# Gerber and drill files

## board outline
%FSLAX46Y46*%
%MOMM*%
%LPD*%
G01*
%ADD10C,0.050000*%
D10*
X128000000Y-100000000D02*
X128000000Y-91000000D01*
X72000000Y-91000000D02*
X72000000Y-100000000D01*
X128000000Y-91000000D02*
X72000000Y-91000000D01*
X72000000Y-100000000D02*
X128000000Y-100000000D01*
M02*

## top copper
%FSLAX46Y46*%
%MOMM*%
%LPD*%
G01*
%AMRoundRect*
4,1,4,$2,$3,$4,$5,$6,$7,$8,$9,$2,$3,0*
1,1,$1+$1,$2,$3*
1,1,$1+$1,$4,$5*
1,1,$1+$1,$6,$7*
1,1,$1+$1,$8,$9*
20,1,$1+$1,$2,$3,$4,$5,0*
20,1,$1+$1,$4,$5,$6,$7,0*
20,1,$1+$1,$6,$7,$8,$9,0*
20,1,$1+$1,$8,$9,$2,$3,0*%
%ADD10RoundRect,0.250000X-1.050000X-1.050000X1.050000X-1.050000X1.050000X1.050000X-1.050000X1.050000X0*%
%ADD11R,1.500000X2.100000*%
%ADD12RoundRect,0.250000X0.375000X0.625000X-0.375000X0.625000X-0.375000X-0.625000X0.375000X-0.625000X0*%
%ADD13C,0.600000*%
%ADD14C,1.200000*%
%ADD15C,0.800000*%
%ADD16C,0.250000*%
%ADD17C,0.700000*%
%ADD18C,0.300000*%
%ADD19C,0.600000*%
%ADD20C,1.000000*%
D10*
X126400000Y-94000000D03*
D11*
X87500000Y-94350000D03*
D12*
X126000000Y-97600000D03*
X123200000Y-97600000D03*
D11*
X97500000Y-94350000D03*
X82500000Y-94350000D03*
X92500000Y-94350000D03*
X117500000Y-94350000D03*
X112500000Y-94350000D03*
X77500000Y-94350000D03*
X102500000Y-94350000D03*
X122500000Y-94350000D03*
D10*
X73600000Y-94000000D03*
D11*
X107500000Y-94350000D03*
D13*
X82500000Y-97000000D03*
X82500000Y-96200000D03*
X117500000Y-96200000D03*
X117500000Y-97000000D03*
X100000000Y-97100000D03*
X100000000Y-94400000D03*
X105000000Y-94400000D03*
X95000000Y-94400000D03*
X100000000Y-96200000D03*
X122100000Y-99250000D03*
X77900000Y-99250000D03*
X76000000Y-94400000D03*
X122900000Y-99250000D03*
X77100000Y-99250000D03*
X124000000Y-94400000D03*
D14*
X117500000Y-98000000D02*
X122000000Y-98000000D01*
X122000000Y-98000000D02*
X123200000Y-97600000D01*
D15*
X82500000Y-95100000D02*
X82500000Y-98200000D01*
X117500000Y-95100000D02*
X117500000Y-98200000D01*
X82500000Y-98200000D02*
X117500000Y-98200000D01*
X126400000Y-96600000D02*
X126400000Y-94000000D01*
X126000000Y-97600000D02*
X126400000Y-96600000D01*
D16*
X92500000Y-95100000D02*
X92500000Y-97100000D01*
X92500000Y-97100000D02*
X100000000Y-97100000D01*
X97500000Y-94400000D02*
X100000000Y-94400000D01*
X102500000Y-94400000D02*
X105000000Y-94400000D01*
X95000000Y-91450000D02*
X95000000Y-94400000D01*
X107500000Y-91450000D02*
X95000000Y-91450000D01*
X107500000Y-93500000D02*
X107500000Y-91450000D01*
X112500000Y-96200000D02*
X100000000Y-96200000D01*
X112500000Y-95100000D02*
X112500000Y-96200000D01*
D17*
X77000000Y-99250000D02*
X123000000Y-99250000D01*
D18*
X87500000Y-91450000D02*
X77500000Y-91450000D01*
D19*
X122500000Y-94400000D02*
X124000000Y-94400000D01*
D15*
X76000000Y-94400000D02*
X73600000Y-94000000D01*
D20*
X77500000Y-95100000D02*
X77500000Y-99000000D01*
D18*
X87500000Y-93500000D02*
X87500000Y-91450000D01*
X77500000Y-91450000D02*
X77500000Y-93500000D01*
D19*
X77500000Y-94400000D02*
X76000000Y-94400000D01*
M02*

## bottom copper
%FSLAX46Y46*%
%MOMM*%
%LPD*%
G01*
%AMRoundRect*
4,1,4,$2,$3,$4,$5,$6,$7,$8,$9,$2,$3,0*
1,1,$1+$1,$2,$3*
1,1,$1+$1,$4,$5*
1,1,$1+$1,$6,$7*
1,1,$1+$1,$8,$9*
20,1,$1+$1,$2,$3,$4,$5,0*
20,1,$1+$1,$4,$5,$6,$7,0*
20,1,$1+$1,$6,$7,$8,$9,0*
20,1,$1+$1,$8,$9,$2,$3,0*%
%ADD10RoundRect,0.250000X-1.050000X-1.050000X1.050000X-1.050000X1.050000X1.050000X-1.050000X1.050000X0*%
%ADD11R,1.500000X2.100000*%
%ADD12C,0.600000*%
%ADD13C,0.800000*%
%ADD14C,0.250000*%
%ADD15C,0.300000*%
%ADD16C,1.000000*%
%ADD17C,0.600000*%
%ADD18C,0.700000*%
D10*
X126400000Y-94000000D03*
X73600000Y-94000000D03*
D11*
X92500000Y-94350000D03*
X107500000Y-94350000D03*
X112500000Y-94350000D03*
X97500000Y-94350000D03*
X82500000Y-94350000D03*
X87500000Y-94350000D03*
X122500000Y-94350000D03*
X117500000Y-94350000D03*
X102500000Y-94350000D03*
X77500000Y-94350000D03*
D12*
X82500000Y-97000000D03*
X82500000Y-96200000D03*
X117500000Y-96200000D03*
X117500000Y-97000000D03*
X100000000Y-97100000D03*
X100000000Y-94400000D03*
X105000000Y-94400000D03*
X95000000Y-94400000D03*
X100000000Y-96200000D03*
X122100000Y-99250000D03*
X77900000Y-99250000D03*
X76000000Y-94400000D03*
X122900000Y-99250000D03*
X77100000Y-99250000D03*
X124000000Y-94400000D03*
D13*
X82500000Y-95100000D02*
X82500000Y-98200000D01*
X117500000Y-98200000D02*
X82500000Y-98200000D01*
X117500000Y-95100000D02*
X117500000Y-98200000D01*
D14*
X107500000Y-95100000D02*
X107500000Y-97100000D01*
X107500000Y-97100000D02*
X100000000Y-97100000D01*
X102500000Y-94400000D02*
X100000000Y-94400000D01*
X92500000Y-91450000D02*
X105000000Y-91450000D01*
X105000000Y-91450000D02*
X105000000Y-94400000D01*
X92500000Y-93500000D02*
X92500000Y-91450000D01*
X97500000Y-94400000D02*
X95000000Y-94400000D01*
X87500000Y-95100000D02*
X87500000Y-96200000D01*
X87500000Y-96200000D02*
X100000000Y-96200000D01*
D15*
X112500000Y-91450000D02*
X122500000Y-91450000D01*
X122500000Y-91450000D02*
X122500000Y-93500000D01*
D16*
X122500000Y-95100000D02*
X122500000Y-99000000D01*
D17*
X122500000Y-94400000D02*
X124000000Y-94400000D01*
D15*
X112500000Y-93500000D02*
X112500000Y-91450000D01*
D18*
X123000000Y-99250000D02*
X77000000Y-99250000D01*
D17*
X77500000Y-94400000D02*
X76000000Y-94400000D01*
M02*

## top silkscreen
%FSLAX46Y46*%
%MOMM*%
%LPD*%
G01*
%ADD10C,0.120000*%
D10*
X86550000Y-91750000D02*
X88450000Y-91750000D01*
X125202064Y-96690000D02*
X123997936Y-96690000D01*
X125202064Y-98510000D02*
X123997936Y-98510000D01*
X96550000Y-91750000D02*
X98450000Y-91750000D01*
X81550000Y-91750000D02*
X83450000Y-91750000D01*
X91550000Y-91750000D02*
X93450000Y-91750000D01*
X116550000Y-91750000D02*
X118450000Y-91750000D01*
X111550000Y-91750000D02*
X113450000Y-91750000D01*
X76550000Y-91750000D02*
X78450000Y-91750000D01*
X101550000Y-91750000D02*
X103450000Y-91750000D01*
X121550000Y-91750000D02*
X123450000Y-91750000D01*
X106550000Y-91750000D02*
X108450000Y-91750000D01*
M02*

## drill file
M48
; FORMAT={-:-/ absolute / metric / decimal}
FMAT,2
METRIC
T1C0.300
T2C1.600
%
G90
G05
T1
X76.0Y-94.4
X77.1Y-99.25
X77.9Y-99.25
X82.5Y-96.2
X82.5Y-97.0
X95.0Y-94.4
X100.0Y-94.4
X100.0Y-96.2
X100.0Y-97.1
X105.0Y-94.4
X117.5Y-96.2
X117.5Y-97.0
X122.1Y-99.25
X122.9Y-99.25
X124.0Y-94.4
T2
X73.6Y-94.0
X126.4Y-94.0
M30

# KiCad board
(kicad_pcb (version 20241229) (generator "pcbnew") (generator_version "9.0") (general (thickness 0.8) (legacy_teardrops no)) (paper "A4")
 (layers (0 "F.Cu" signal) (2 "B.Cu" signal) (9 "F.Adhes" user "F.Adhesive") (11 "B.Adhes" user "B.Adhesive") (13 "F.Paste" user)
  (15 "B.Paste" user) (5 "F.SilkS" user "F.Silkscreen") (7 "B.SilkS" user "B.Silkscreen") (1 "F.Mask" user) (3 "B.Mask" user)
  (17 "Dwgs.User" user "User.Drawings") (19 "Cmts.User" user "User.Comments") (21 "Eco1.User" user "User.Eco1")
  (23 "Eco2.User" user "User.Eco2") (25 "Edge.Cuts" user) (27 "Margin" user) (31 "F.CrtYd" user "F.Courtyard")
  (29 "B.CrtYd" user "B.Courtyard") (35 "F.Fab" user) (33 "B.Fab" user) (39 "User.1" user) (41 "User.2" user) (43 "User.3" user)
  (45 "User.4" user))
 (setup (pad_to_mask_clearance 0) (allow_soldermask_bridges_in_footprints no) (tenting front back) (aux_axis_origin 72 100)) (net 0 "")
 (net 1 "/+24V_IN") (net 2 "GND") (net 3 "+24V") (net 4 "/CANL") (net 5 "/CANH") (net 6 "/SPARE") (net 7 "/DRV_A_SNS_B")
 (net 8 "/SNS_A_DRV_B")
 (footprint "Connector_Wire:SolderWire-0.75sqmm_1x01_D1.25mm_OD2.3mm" (layer "F.Cu") (at 126.4 94)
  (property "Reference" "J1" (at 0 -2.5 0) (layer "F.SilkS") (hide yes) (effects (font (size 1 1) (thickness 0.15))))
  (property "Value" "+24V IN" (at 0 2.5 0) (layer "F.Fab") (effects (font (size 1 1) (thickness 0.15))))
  (pad "1" thru_hole roundrect (at 0 0) (size 2.6 2.6) (drill 1.6) (layers "*.Cu" "*.Mask") (remove_unused_layers no)
   (roundrect_rratio 0.096154) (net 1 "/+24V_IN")))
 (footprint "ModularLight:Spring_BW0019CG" (layer "F.Cu") (at 87.5 93.65)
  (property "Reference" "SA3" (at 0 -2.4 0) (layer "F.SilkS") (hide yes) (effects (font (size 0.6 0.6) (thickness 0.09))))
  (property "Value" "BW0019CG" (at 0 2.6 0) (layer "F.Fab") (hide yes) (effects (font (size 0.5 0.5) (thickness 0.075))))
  (fp_line (start -0.95 -1.9) (end 0.95 -1.9) (stroke (width 0.12) (type solid)) (layer "F.SilkS"))
  (pad "1" smd rect (at 0 0.7) (size 1.5 2.1) (layers "F.Cu" "F.Mask" "F.Paste") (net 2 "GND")))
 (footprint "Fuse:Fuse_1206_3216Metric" (layer "F.Cu") (at 124.6 97.6 180)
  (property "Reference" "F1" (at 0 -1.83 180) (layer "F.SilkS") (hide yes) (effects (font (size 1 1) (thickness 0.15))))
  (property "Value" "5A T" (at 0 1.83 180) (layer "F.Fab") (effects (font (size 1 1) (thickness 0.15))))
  (fp_line (start -0.602064 0.91) (end 0.602064 0.91) (stroke (width 0.12) (type solid)) (layer "F.SilkS"))
  (fp_line (start -0.602064 -0.91) (end 0.602064 -0.91) (stroke (width 0.12) (type solid)) (layer "F.SilkS"))
  (pad "1" smd roundrect (at -1.4 0 180) (size 1.25 1.75) (layers "F.Cu" "F.Mask" "F.Paste") (roundrect_rratio 0.2) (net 1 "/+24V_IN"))
  (pad "2" smd roundrect (at 1.4 0 180) (size 1.25 1.75) (layers "F.Cu" "F.Mask" "F.Paste") (roundrect_rratio 0.2) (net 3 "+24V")))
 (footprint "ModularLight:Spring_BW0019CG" (layer "F.Cu") (at 97.5 93.65)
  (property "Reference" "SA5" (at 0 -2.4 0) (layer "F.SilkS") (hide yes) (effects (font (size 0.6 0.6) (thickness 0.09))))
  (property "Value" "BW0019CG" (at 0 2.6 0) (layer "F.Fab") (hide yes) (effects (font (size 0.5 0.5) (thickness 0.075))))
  (fp_line (start -0.95 -1.9) (end 0.95 -1.9) (stroke (width 0.12) (type solid)) (layer "F.SilkS"))
  (pad "1" smd rect (at 0 0.7) (size 1.5 2.1) (layers "F.Cu" "F.Mask" "F.Paste") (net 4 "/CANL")))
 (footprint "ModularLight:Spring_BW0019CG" (layer "F.Cu") (at 82.5 93.65)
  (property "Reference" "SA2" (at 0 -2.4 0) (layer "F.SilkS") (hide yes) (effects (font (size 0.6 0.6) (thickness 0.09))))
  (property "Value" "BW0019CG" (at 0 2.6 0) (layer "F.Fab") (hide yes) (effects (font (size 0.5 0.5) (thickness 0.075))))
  (fp_line (start -0.95 -1.9) (end 0.95 -1.9) (stroke (width 0.12) (type solid)) (layer "F.SilkS"))
  (pad "1" smd rect (at 0 0.7) (size 1.5 2.1) (layers "F.Cu" "F.Mask" "F.Paste") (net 3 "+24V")))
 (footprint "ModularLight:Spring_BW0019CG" (layer "F.Cu") (at 92.5 93.65)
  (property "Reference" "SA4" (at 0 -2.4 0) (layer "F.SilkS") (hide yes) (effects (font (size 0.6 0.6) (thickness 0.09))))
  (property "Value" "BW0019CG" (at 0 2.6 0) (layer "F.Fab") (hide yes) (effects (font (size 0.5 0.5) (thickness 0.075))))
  (fp_line (start -0.95 -1.9) (end 0.95 -1.9) (stroke (width 0.12) (type solid)) (layer "F.SilkS"))
  (pad "1" smd rect (at 0 0.7) (size 1.5 2.1) (layers "F.Cu" "F.Mask" "F.Paste") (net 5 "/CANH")))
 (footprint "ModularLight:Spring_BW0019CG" (layer "F.Cu") (at 117.5 93.65)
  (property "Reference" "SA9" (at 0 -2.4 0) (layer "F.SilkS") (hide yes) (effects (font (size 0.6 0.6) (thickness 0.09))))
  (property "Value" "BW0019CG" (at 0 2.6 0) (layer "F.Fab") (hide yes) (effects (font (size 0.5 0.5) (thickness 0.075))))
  (fp_line (start -0.95 -1.9) (end 0.95 -1.9) (stroke (width 0.12) (type solid)) (layer "F.SilkS"))
  (pad "1" smd rect (at 0 0.7) (size 1.5 2.1) (layers "F.Cu" "F.Mask" "F.Paste") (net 3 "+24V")))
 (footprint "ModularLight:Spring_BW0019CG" (layer "F.Cu") (at 112.5 93.65)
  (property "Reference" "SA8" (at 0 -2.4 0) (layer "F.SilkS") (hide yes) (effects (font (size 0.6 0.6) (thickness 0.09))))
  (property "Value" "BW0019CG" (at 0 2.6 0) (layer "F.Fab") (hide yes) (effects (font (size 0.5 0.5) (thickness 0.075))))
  (fp_line (start -0.95 -1.9) (end 0.95 -1.9) (stroke (width 0.12) (type solid)) (layer "F.SilkS"))
  (pad "1" smd rect (at 0 0.7) (size 1.5 2.1) (layers "F.Cu" "F.Mask" "F.Paste") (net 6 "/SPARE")))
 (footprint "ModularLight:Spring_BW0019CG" (layer "F.Cu") (at 77.5 93.65)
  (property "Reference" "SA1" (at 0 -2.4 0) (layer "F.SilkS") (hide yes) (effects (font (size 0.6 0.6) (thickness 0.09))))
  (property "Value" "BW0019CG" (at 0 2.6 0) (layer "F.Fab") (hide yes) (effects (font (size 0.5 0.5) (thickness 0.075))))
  (fp_line (start -0.95 -1.9) (end 0.95 -1.9) (stroke (width 0.12) (type solid)) (layer "F.SilkS"))
  (pad "1" smd rect (at 0 0.7) (size 1.5 2.1) (layers "F.Cu" "F.Mask" "F.Paste") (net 2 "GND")))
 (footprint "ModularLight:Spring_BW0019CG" (layer "F.Cu") (at 102.5 93.65)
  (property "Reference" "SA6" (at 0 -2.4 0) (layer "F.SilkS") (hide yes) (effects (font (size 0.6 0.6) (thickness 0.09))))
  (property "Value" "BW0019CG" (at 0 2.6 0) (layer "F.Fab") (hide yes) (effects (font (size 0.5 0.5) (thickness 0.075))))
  (fp_line (start -0.95 -1.9) (end 0.95 -1.9) (stroke (width 0.12) (type solid)) (layer "F.SilkS"))
  (pad "1" smd rect (at 0 0.7) (size 1.5 2.1) (layers "F.Cu" "F.Mask" "F.Paste") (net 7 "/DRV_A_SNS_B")))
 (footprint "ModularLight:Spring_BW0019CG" (layer "F.Cu") (at 122.5 93.65)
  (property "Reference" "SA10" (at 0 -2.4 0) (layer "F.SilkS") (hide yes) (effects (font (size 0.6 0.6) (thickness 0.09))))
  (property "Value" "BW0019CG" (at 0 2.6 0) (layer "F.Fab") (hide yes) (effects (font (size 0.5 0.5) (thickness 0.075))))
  (fp_line (start -0.95 -1.9) (end 0.95 -1.9) (stroke (width 0.12) (type solid)) (layer "F.SilkS"))
  (pad "1" smd rect (at 0 0.7) (size 1.5 2.1) (layers "F.Cu" "F.Mask" "F.Paste") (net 2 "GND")))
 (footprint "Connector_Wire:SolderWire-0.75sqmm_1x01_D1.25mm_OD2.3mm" (layer "F.Cu") (at 73.6 94)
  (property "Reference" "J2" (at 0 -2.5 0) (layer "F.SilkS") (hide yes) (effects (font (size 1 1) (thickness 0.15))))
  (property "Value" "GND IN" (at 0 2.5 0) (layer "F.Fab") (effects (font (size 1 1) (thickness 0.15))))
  (pad "1" thru_hole roundrect (at 0 0) (size 2.6 2.6) (drill 1.6) (layers "*.Cu" "*.Mask") (remove_unused_layers no)
   (roundrect_rratio 0.096154) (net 2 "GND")))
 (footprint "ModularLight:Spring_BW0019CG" (layer "F.Cu") (at 107.5 93.65)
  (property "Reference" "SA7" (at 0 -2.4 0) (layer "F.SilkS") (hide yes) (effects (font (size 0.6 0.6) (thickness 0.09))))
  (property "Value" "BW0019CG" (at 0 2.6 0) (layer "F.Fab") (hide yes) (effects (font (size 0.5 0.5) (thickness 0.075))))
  (fp_line (start -0.95 -1.9) (end 0.95 -1.9) (stroke (width 0.12) (type solid)) (layer "F.SilkS"))
  (pad "1" smd rect (at 0 0.7) (size 1.5 2.1) (layers "F.Cu" "F.Mask" "F.Paste") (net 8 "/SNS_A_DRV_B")))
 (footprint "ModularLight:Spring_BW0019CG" (layer "B.Cu") (at 92.5 93.65 180)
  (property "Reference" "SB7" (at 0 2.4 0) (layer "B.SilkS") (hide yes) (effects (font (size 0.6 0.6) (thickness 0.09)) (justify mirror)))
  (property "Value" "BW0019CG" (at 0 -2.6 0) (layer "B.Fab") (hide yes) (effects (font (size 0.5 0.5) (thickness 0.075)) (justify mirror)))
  (pad "1" smd rect (at 0 -0.7 180) (size 1.5 2.1) (layers "B.Cu" "B.Mask" "B.Paste") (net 7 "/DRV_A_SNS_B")))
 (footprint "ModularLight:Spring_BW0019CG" (layer "B.Cu") (at 107.5 93.65 180)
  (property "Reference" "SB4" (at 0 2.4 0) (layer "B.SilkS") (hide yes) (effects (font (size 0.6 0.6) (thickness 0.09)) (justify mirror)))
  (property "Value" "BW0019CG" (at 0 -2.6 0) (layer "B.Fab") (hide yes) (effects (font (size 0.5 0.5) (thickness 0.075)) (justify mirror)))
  (pad "1" smd rect (at 0 -0.7 180) (size 1.5 2.1) (layers "B.Cu" "B.Mask" "B.Paste") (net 5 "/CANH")))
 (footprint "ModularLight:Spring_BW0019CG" (layer "B.Cu") (at 112.5 93.65 180)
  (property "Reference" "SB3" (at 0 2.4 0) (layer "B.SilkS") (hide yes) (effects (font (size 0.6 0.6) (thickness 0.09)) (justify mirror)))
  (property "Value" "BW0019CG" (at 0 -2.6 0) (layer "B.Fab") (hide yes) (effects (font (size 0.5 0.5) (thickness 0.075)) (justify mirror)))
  (pad "1" smd rect (at 0 -0.7 180) (size 1.5 2.1) (layers "B.Cu" "B.Mask" "B.Paste") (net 2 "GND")))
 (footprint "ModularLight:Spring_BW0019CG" (layer "B.Cu") (at 97.5 93.65 180)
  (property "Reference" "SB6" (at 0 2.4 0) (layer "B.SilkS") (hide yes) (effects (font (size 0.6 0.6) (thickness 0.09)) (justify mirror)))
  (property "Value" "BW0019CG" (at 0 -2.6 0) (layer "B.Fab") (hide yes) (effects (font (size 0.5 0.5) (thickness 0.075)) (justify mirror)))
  (pad "1" smd rect (at 0 -0.7 180) (size 1.5 2.1) (layers "B.Cu" "B.Mask" "B.Paste") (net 8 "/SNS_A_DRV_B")))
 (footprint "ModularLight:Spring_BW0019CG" (layer "B.Cu") (at 82.5 93.65 180)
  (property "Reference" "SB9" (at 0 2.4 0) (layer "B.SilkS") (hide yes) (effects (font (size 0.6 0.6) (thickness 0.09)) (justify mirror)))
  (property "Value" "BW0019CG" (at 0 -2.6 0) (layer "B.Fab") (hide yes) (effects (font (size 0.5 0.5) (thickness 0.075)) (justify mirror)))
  (pad "1" smd rect (at 0 -0.7 180) (size 1.5 2.1) (layers "B.Cu" "B.Mask" "B.Paste") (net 3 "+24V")))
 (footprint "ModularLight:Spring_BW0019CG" (layer "B.Cu") (at 87.5 93.65 180)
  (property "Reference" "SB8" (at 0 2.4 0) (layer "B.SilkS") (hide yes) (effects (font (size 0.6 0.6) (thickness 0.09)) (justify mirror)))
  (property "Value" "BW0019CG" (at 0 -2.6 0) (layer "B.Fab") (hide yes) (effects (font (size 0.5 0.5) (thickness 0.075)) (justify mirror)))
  (pad "1" smd rect (at 0 -0.7 180) (size 1.5 2.1) (layers "B.Cu" "B.Mask" "B.Paste") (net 6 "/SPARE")))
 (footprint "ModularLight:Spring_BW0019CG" (layer "B.Cu") (at 122.5 93.65 180)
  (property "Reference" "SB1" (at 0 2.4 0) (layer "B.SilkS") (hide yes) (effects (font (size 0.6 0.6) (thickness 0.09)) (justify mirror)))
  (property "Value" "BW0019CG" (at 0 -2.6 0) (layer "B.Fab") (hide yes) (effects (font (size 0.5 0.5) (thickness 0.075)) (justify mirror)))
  (pad "1" smd rect (at 0 -0.7 180) (size 1.5 2.1) (layers "B.Cu" "B.Mask" "B.Paste") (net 2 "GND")))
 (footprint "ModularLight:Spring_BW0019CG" (layer "B.Cu") (at 117.5 93.65 180)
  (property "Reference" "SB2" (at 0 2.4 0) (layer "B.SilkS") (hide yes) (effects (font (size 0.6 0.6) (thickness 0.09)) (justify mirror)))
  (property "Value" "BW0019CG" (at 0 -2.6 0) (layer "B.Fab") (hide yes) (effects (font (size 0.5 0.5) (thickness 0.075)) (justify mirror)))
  (pad "1" smd rect (at 0 -0.7 180) (size 1.5 2.1) (layers "B.Cu" "B.Mask" "B.Paste") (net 3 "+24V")))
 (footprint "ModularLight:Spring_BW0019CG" (layer "B.Cu") (at 102.5 93.65 180)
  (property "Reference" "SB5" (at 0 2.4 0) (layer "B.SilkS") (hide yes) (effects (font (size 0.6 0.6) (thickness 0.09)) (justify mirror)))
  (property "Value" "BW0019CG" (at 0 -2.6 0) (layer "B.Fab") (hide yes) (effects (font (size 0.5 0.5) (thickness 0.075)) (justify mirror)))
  (pad "1" smd rect (at 0 -0.7 180) (size 1.5 2.1) (layers "B.Cu" "B.Mask" "B.Paste") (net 4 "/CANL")))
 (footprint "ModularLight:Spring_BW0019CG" (layer "B.Cu") (at 77.5 93.65 180)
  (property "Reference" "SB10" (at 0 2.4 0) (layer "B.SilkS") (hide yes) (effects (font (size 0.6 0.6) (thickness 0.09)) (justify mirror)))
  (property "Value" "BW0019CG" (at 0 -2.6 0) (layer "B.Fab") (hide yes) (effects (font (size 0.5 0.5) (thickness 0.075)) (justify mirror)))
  (pad "1" smd rect (at 0 -0.7 180) (size 1.5 2.1) (layers "B.Cu" "B.Mask" "B.Paste") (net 2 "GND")))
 (gr_line (start 128 100) (end 128 91) (stroke (width 0.05) (type default)) (layer "Edge.Cuts"))
 (gr_line (start 72 91) (end 72 100) (stroke (width 0.05) (type default)) (layer "Edge.Cuts"))
 (gr_line (start 128 91) (end 72 91) (stroke (width 0.05) (type default)) (layer "Edge.Cuts"))
 (gr_line (start 72 100) (end 128 100) (stroke (width 0.05) (type default)) (layer "Edge.Cuts"))
 (segment (start 117.5 98) (end 122 98) (width 1.2) (locked yes) (layer "F.Cu") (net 3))
 (segment (start 122 98) (end 123.2 97.6) (width 1.2) (locked yes) (layer "F.Cu") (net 3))
 (segment (start 82.5 95.1) (end 82.5 98.2) (width 0.8) (locked yes) (layer "F.Cu") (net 3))
 (segment (start 117.5 95.1) (end 117.5 98.2) (width 0.8) (locked yes) (layer "F.Cu") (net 3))
 (segment (start 82.5 98.2) (end 117.5 98.2) (width 0.8) (locked yes) (layer "F.Cu") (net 3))
 (via (at 82.5 97) (size 0.6) (drill 0.3) (layers "F.Cu" "B.Cu") (locked yes) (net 3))
 (via (at 82.5 96.2) (size 0.6) (drill 0.3) (layers "F.Cu" "B.Cu") (locked yes) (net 3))
 (via (at 117.5 96.2) (size 0.6) (drill 0.3) (layers "F.Cu" "B.Cu") (locked yes) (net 3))
 (via (at 117.5 97) (size 0.6) (drill 0.3) (layers "F.Cu" "B.Cu") (locked yes) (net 3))
 (segment (start 82.5 95.1) (end 82.5 98.2) (width 0.8) (locked yes) (layer "B.Cu") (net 3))
 (segment (start 117.5 98.2) (end 82.5 98.2) (width 0.8) (locked yes) (layer "B.Cu") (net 3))
 (segment (start 117.5 95.1) (end 117.5 98.2) (width 0.8) (locked yes) (layer "B.Cu") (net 3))
 (segment (start 126.4 96.6) (end 126.4 94) (width 0.8) (locked yes) (layer "F.Cu") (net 1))
 (segment (start 126 97.6) (end 126.4 96.6) (width 0.8) (locked yes) (layer "F.Cu") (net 1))
 (segment (start 92.5 95.1) (end 92.5 97.1) (width 0.25) (locked yes) (layer "F.Cu") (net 5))
 (segment (start 92.5 97.1) (end 100 97.1) (width 0.25) (locked yes) (layer "F.Cu") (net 5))
 (via (at 100 97.1) (size 0.6) (drill 0.3) (layers "F.Cu" "B.Cu") (locked yes) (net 5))
 (segment (start 107.5 95.1) (end 107.5 97.1) (width 0.25) (locked yes) (layer "B.Cu") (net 5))
 (segment (start 107.5 97.1) (end 100 97.1) (width 0.25) (locked yes) (layer "B.Cu") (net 5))
 (segment (start 97.5 94.4) (end 100 94.4) (width 0.25) (locked yes) (layer "F.Cu") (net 4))
 (via (at 100 94.4) (size 0.6) (drill 0.3) (layers "F.Cu" "B.Cu") (locked yes) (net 4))
 (segment (start 102.5 94.4) (end 100 94.4) (width 0.25) (locked yes) (layer "B.Cu") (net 4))
 (segment (start 102.5 94.4) (end 105 94.4) (width 0.25) (locked yes) (layer "F.Cu") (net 7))
 (via (at 105 94.4) (size 0.6) (drill 0.3) (layers "F.Cu" "B.Cu") (locked yes) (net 7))
 (segment (start 92.5 91.45) (end 105 91.45) (width 0.25) (locked yes) (layer "B.Cu") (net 7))
 (segment (start 105 91.45) (end 105 94.4) (width 0.25) (locked yes) (layer "B.Cu") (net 7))
 (segment (start 92.5 93.5) (end 92.5 91.45) (width 0.25) (locked yes) (layer "B.Cu") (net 7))
 (segment (start 95 91.45) (end 95 94.4) (width 0.25) (locked yes) (layer "F.Cu") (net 8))
 (segment (start 107.5 91.45) (end 95 91.45) (width 0.25) (locked yes) (layer "F.Cu") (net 8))
 (segment (start 107.5 93.5) (end 107.5 91.45) (width 0.25) (locked yes) (layer "F.Cu") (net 8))
 (via (at 95 94.4) (size 0.6) (drill 0.3) (layers "F.Cu" "B.Cu") (locked yes) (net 8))
 (segment (start 97.5 94.4) (end 95 94.4) (width 0.25) (locked yes) (layer "B.Cu") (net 8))
 (segment (start 112.5 96.2) (end 100 96.2) (width 0.25) (locked yes) (layer "F.Cu") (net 6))
 (segment (start 112.5 95.1) (end 112.5 96.2) (width 0.25) (locked yes) (layer "F.Cu") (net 6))
 (via (at 100 96.2) (size 0.6) (drill 0.3) (layers "F.Cu" "B.Cu") (locked yes) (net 6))
 (segment (start 87.5 95.1) (end 87.5 96.2) (width 0.25) (locked yes) (layer "B.Cu") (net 6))
 (segment (start 87.5 96.2) (end 100 96.2) (width 0.25) (locked yes) (layer "B.Cu") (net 6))
 (segment (start 77 99.25) (end 123 99.25) (width 0.7) (locked yes) (layer "F.Cu") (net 2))
 (segment (start 87.5 91.45) (end 77.5 91.45) (width 0.3) (locked yes) (layer "F.Cu") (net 2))
 (segment (start 122.5 94.4) (end 124 94.4) (width 0.6) (locked yes) (layer "F.Cu") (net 2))
 (segment (start 76 94.4) (end 73.6 94) (width 0.8) (locked yes) (layer "F.Cu") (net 2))
 (segment (start 77.5 95.1) (end 77.5 99) (width 1) (locked yes) (layer "F.Cu") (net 2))
 (segment (start 87.5 93.5) (end 87.5 91.45) (width 0.3) (locked yes) (layer "F.Cu") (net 2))
 (segment (start 77.5 91.45) (end 77.5 93.5) (width 0.3) (locked yes) (layer "F.Cu") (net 2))
 (segment (start 77.5 94.4) (end 76 94.4) (width 0.6) (locked yes) (layer "F.Cu") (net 2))
 (via (at 122.1 99.25) (size 0.6) (drill 0.3) (layers "F.Cu" "B.Cu") (locked yes) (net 2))
 (via (at 77.9 99.25) (size 0.6) (drill 0.3) (layers "F.Cu" "B.Cu") (locked yes) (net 2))
 (via (at 76 94.4) (size 0.6) (drill 0.3) (layers "F.Cu" "B.Cu") (locked yes) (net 2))
 (via (at 122.9 99.25) (size 0.6) (drill 0.3) (layers "F.Cu" "B.Cu") (locked yes) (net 2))
 (via (at 77.1 99.25) (size 0.6) (drill 0.3) (layers "F.Cu" "B.Cu") (locked yes) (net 2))
 (via (at 124 94.4) (size 0.6) (drill 0.3) (layers "F.Cu" "B.Cu") (locked yes) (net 2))
 (segment (start 112.5 91.45) (end 122.5 91.45) (width 0.3) (locked yes) (layer "B.Cu") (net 2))
 (segment (start 122.5 91.45) (end 122.5 93.5) (width 0.3) (locked yes) (layer "B.Cu") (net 2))
 (segment (start 122.5 95.1) (end 122.5 99) (width 1) (locked yes) (layer "B.Cu") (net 2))
 (segment (start 122.5 94.4) (end 124 94.4) (width 0.6) (locked yes) (layer "B.Cu") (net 2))
 (segment (start 112.5 93.5) (end 112.5 91.45) (width 0.3) (locked yes) (layer "B.Cu") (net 2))
 (segment (start 123 99.25) (end 77 99.25) (width 0.7) (locked yes) (layer "B.Cu") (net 2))
 (segment (start 77.5 94.4) (end 76 94.4) (width 0.6) (locked yes) (layer "B.Cu") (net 2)))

